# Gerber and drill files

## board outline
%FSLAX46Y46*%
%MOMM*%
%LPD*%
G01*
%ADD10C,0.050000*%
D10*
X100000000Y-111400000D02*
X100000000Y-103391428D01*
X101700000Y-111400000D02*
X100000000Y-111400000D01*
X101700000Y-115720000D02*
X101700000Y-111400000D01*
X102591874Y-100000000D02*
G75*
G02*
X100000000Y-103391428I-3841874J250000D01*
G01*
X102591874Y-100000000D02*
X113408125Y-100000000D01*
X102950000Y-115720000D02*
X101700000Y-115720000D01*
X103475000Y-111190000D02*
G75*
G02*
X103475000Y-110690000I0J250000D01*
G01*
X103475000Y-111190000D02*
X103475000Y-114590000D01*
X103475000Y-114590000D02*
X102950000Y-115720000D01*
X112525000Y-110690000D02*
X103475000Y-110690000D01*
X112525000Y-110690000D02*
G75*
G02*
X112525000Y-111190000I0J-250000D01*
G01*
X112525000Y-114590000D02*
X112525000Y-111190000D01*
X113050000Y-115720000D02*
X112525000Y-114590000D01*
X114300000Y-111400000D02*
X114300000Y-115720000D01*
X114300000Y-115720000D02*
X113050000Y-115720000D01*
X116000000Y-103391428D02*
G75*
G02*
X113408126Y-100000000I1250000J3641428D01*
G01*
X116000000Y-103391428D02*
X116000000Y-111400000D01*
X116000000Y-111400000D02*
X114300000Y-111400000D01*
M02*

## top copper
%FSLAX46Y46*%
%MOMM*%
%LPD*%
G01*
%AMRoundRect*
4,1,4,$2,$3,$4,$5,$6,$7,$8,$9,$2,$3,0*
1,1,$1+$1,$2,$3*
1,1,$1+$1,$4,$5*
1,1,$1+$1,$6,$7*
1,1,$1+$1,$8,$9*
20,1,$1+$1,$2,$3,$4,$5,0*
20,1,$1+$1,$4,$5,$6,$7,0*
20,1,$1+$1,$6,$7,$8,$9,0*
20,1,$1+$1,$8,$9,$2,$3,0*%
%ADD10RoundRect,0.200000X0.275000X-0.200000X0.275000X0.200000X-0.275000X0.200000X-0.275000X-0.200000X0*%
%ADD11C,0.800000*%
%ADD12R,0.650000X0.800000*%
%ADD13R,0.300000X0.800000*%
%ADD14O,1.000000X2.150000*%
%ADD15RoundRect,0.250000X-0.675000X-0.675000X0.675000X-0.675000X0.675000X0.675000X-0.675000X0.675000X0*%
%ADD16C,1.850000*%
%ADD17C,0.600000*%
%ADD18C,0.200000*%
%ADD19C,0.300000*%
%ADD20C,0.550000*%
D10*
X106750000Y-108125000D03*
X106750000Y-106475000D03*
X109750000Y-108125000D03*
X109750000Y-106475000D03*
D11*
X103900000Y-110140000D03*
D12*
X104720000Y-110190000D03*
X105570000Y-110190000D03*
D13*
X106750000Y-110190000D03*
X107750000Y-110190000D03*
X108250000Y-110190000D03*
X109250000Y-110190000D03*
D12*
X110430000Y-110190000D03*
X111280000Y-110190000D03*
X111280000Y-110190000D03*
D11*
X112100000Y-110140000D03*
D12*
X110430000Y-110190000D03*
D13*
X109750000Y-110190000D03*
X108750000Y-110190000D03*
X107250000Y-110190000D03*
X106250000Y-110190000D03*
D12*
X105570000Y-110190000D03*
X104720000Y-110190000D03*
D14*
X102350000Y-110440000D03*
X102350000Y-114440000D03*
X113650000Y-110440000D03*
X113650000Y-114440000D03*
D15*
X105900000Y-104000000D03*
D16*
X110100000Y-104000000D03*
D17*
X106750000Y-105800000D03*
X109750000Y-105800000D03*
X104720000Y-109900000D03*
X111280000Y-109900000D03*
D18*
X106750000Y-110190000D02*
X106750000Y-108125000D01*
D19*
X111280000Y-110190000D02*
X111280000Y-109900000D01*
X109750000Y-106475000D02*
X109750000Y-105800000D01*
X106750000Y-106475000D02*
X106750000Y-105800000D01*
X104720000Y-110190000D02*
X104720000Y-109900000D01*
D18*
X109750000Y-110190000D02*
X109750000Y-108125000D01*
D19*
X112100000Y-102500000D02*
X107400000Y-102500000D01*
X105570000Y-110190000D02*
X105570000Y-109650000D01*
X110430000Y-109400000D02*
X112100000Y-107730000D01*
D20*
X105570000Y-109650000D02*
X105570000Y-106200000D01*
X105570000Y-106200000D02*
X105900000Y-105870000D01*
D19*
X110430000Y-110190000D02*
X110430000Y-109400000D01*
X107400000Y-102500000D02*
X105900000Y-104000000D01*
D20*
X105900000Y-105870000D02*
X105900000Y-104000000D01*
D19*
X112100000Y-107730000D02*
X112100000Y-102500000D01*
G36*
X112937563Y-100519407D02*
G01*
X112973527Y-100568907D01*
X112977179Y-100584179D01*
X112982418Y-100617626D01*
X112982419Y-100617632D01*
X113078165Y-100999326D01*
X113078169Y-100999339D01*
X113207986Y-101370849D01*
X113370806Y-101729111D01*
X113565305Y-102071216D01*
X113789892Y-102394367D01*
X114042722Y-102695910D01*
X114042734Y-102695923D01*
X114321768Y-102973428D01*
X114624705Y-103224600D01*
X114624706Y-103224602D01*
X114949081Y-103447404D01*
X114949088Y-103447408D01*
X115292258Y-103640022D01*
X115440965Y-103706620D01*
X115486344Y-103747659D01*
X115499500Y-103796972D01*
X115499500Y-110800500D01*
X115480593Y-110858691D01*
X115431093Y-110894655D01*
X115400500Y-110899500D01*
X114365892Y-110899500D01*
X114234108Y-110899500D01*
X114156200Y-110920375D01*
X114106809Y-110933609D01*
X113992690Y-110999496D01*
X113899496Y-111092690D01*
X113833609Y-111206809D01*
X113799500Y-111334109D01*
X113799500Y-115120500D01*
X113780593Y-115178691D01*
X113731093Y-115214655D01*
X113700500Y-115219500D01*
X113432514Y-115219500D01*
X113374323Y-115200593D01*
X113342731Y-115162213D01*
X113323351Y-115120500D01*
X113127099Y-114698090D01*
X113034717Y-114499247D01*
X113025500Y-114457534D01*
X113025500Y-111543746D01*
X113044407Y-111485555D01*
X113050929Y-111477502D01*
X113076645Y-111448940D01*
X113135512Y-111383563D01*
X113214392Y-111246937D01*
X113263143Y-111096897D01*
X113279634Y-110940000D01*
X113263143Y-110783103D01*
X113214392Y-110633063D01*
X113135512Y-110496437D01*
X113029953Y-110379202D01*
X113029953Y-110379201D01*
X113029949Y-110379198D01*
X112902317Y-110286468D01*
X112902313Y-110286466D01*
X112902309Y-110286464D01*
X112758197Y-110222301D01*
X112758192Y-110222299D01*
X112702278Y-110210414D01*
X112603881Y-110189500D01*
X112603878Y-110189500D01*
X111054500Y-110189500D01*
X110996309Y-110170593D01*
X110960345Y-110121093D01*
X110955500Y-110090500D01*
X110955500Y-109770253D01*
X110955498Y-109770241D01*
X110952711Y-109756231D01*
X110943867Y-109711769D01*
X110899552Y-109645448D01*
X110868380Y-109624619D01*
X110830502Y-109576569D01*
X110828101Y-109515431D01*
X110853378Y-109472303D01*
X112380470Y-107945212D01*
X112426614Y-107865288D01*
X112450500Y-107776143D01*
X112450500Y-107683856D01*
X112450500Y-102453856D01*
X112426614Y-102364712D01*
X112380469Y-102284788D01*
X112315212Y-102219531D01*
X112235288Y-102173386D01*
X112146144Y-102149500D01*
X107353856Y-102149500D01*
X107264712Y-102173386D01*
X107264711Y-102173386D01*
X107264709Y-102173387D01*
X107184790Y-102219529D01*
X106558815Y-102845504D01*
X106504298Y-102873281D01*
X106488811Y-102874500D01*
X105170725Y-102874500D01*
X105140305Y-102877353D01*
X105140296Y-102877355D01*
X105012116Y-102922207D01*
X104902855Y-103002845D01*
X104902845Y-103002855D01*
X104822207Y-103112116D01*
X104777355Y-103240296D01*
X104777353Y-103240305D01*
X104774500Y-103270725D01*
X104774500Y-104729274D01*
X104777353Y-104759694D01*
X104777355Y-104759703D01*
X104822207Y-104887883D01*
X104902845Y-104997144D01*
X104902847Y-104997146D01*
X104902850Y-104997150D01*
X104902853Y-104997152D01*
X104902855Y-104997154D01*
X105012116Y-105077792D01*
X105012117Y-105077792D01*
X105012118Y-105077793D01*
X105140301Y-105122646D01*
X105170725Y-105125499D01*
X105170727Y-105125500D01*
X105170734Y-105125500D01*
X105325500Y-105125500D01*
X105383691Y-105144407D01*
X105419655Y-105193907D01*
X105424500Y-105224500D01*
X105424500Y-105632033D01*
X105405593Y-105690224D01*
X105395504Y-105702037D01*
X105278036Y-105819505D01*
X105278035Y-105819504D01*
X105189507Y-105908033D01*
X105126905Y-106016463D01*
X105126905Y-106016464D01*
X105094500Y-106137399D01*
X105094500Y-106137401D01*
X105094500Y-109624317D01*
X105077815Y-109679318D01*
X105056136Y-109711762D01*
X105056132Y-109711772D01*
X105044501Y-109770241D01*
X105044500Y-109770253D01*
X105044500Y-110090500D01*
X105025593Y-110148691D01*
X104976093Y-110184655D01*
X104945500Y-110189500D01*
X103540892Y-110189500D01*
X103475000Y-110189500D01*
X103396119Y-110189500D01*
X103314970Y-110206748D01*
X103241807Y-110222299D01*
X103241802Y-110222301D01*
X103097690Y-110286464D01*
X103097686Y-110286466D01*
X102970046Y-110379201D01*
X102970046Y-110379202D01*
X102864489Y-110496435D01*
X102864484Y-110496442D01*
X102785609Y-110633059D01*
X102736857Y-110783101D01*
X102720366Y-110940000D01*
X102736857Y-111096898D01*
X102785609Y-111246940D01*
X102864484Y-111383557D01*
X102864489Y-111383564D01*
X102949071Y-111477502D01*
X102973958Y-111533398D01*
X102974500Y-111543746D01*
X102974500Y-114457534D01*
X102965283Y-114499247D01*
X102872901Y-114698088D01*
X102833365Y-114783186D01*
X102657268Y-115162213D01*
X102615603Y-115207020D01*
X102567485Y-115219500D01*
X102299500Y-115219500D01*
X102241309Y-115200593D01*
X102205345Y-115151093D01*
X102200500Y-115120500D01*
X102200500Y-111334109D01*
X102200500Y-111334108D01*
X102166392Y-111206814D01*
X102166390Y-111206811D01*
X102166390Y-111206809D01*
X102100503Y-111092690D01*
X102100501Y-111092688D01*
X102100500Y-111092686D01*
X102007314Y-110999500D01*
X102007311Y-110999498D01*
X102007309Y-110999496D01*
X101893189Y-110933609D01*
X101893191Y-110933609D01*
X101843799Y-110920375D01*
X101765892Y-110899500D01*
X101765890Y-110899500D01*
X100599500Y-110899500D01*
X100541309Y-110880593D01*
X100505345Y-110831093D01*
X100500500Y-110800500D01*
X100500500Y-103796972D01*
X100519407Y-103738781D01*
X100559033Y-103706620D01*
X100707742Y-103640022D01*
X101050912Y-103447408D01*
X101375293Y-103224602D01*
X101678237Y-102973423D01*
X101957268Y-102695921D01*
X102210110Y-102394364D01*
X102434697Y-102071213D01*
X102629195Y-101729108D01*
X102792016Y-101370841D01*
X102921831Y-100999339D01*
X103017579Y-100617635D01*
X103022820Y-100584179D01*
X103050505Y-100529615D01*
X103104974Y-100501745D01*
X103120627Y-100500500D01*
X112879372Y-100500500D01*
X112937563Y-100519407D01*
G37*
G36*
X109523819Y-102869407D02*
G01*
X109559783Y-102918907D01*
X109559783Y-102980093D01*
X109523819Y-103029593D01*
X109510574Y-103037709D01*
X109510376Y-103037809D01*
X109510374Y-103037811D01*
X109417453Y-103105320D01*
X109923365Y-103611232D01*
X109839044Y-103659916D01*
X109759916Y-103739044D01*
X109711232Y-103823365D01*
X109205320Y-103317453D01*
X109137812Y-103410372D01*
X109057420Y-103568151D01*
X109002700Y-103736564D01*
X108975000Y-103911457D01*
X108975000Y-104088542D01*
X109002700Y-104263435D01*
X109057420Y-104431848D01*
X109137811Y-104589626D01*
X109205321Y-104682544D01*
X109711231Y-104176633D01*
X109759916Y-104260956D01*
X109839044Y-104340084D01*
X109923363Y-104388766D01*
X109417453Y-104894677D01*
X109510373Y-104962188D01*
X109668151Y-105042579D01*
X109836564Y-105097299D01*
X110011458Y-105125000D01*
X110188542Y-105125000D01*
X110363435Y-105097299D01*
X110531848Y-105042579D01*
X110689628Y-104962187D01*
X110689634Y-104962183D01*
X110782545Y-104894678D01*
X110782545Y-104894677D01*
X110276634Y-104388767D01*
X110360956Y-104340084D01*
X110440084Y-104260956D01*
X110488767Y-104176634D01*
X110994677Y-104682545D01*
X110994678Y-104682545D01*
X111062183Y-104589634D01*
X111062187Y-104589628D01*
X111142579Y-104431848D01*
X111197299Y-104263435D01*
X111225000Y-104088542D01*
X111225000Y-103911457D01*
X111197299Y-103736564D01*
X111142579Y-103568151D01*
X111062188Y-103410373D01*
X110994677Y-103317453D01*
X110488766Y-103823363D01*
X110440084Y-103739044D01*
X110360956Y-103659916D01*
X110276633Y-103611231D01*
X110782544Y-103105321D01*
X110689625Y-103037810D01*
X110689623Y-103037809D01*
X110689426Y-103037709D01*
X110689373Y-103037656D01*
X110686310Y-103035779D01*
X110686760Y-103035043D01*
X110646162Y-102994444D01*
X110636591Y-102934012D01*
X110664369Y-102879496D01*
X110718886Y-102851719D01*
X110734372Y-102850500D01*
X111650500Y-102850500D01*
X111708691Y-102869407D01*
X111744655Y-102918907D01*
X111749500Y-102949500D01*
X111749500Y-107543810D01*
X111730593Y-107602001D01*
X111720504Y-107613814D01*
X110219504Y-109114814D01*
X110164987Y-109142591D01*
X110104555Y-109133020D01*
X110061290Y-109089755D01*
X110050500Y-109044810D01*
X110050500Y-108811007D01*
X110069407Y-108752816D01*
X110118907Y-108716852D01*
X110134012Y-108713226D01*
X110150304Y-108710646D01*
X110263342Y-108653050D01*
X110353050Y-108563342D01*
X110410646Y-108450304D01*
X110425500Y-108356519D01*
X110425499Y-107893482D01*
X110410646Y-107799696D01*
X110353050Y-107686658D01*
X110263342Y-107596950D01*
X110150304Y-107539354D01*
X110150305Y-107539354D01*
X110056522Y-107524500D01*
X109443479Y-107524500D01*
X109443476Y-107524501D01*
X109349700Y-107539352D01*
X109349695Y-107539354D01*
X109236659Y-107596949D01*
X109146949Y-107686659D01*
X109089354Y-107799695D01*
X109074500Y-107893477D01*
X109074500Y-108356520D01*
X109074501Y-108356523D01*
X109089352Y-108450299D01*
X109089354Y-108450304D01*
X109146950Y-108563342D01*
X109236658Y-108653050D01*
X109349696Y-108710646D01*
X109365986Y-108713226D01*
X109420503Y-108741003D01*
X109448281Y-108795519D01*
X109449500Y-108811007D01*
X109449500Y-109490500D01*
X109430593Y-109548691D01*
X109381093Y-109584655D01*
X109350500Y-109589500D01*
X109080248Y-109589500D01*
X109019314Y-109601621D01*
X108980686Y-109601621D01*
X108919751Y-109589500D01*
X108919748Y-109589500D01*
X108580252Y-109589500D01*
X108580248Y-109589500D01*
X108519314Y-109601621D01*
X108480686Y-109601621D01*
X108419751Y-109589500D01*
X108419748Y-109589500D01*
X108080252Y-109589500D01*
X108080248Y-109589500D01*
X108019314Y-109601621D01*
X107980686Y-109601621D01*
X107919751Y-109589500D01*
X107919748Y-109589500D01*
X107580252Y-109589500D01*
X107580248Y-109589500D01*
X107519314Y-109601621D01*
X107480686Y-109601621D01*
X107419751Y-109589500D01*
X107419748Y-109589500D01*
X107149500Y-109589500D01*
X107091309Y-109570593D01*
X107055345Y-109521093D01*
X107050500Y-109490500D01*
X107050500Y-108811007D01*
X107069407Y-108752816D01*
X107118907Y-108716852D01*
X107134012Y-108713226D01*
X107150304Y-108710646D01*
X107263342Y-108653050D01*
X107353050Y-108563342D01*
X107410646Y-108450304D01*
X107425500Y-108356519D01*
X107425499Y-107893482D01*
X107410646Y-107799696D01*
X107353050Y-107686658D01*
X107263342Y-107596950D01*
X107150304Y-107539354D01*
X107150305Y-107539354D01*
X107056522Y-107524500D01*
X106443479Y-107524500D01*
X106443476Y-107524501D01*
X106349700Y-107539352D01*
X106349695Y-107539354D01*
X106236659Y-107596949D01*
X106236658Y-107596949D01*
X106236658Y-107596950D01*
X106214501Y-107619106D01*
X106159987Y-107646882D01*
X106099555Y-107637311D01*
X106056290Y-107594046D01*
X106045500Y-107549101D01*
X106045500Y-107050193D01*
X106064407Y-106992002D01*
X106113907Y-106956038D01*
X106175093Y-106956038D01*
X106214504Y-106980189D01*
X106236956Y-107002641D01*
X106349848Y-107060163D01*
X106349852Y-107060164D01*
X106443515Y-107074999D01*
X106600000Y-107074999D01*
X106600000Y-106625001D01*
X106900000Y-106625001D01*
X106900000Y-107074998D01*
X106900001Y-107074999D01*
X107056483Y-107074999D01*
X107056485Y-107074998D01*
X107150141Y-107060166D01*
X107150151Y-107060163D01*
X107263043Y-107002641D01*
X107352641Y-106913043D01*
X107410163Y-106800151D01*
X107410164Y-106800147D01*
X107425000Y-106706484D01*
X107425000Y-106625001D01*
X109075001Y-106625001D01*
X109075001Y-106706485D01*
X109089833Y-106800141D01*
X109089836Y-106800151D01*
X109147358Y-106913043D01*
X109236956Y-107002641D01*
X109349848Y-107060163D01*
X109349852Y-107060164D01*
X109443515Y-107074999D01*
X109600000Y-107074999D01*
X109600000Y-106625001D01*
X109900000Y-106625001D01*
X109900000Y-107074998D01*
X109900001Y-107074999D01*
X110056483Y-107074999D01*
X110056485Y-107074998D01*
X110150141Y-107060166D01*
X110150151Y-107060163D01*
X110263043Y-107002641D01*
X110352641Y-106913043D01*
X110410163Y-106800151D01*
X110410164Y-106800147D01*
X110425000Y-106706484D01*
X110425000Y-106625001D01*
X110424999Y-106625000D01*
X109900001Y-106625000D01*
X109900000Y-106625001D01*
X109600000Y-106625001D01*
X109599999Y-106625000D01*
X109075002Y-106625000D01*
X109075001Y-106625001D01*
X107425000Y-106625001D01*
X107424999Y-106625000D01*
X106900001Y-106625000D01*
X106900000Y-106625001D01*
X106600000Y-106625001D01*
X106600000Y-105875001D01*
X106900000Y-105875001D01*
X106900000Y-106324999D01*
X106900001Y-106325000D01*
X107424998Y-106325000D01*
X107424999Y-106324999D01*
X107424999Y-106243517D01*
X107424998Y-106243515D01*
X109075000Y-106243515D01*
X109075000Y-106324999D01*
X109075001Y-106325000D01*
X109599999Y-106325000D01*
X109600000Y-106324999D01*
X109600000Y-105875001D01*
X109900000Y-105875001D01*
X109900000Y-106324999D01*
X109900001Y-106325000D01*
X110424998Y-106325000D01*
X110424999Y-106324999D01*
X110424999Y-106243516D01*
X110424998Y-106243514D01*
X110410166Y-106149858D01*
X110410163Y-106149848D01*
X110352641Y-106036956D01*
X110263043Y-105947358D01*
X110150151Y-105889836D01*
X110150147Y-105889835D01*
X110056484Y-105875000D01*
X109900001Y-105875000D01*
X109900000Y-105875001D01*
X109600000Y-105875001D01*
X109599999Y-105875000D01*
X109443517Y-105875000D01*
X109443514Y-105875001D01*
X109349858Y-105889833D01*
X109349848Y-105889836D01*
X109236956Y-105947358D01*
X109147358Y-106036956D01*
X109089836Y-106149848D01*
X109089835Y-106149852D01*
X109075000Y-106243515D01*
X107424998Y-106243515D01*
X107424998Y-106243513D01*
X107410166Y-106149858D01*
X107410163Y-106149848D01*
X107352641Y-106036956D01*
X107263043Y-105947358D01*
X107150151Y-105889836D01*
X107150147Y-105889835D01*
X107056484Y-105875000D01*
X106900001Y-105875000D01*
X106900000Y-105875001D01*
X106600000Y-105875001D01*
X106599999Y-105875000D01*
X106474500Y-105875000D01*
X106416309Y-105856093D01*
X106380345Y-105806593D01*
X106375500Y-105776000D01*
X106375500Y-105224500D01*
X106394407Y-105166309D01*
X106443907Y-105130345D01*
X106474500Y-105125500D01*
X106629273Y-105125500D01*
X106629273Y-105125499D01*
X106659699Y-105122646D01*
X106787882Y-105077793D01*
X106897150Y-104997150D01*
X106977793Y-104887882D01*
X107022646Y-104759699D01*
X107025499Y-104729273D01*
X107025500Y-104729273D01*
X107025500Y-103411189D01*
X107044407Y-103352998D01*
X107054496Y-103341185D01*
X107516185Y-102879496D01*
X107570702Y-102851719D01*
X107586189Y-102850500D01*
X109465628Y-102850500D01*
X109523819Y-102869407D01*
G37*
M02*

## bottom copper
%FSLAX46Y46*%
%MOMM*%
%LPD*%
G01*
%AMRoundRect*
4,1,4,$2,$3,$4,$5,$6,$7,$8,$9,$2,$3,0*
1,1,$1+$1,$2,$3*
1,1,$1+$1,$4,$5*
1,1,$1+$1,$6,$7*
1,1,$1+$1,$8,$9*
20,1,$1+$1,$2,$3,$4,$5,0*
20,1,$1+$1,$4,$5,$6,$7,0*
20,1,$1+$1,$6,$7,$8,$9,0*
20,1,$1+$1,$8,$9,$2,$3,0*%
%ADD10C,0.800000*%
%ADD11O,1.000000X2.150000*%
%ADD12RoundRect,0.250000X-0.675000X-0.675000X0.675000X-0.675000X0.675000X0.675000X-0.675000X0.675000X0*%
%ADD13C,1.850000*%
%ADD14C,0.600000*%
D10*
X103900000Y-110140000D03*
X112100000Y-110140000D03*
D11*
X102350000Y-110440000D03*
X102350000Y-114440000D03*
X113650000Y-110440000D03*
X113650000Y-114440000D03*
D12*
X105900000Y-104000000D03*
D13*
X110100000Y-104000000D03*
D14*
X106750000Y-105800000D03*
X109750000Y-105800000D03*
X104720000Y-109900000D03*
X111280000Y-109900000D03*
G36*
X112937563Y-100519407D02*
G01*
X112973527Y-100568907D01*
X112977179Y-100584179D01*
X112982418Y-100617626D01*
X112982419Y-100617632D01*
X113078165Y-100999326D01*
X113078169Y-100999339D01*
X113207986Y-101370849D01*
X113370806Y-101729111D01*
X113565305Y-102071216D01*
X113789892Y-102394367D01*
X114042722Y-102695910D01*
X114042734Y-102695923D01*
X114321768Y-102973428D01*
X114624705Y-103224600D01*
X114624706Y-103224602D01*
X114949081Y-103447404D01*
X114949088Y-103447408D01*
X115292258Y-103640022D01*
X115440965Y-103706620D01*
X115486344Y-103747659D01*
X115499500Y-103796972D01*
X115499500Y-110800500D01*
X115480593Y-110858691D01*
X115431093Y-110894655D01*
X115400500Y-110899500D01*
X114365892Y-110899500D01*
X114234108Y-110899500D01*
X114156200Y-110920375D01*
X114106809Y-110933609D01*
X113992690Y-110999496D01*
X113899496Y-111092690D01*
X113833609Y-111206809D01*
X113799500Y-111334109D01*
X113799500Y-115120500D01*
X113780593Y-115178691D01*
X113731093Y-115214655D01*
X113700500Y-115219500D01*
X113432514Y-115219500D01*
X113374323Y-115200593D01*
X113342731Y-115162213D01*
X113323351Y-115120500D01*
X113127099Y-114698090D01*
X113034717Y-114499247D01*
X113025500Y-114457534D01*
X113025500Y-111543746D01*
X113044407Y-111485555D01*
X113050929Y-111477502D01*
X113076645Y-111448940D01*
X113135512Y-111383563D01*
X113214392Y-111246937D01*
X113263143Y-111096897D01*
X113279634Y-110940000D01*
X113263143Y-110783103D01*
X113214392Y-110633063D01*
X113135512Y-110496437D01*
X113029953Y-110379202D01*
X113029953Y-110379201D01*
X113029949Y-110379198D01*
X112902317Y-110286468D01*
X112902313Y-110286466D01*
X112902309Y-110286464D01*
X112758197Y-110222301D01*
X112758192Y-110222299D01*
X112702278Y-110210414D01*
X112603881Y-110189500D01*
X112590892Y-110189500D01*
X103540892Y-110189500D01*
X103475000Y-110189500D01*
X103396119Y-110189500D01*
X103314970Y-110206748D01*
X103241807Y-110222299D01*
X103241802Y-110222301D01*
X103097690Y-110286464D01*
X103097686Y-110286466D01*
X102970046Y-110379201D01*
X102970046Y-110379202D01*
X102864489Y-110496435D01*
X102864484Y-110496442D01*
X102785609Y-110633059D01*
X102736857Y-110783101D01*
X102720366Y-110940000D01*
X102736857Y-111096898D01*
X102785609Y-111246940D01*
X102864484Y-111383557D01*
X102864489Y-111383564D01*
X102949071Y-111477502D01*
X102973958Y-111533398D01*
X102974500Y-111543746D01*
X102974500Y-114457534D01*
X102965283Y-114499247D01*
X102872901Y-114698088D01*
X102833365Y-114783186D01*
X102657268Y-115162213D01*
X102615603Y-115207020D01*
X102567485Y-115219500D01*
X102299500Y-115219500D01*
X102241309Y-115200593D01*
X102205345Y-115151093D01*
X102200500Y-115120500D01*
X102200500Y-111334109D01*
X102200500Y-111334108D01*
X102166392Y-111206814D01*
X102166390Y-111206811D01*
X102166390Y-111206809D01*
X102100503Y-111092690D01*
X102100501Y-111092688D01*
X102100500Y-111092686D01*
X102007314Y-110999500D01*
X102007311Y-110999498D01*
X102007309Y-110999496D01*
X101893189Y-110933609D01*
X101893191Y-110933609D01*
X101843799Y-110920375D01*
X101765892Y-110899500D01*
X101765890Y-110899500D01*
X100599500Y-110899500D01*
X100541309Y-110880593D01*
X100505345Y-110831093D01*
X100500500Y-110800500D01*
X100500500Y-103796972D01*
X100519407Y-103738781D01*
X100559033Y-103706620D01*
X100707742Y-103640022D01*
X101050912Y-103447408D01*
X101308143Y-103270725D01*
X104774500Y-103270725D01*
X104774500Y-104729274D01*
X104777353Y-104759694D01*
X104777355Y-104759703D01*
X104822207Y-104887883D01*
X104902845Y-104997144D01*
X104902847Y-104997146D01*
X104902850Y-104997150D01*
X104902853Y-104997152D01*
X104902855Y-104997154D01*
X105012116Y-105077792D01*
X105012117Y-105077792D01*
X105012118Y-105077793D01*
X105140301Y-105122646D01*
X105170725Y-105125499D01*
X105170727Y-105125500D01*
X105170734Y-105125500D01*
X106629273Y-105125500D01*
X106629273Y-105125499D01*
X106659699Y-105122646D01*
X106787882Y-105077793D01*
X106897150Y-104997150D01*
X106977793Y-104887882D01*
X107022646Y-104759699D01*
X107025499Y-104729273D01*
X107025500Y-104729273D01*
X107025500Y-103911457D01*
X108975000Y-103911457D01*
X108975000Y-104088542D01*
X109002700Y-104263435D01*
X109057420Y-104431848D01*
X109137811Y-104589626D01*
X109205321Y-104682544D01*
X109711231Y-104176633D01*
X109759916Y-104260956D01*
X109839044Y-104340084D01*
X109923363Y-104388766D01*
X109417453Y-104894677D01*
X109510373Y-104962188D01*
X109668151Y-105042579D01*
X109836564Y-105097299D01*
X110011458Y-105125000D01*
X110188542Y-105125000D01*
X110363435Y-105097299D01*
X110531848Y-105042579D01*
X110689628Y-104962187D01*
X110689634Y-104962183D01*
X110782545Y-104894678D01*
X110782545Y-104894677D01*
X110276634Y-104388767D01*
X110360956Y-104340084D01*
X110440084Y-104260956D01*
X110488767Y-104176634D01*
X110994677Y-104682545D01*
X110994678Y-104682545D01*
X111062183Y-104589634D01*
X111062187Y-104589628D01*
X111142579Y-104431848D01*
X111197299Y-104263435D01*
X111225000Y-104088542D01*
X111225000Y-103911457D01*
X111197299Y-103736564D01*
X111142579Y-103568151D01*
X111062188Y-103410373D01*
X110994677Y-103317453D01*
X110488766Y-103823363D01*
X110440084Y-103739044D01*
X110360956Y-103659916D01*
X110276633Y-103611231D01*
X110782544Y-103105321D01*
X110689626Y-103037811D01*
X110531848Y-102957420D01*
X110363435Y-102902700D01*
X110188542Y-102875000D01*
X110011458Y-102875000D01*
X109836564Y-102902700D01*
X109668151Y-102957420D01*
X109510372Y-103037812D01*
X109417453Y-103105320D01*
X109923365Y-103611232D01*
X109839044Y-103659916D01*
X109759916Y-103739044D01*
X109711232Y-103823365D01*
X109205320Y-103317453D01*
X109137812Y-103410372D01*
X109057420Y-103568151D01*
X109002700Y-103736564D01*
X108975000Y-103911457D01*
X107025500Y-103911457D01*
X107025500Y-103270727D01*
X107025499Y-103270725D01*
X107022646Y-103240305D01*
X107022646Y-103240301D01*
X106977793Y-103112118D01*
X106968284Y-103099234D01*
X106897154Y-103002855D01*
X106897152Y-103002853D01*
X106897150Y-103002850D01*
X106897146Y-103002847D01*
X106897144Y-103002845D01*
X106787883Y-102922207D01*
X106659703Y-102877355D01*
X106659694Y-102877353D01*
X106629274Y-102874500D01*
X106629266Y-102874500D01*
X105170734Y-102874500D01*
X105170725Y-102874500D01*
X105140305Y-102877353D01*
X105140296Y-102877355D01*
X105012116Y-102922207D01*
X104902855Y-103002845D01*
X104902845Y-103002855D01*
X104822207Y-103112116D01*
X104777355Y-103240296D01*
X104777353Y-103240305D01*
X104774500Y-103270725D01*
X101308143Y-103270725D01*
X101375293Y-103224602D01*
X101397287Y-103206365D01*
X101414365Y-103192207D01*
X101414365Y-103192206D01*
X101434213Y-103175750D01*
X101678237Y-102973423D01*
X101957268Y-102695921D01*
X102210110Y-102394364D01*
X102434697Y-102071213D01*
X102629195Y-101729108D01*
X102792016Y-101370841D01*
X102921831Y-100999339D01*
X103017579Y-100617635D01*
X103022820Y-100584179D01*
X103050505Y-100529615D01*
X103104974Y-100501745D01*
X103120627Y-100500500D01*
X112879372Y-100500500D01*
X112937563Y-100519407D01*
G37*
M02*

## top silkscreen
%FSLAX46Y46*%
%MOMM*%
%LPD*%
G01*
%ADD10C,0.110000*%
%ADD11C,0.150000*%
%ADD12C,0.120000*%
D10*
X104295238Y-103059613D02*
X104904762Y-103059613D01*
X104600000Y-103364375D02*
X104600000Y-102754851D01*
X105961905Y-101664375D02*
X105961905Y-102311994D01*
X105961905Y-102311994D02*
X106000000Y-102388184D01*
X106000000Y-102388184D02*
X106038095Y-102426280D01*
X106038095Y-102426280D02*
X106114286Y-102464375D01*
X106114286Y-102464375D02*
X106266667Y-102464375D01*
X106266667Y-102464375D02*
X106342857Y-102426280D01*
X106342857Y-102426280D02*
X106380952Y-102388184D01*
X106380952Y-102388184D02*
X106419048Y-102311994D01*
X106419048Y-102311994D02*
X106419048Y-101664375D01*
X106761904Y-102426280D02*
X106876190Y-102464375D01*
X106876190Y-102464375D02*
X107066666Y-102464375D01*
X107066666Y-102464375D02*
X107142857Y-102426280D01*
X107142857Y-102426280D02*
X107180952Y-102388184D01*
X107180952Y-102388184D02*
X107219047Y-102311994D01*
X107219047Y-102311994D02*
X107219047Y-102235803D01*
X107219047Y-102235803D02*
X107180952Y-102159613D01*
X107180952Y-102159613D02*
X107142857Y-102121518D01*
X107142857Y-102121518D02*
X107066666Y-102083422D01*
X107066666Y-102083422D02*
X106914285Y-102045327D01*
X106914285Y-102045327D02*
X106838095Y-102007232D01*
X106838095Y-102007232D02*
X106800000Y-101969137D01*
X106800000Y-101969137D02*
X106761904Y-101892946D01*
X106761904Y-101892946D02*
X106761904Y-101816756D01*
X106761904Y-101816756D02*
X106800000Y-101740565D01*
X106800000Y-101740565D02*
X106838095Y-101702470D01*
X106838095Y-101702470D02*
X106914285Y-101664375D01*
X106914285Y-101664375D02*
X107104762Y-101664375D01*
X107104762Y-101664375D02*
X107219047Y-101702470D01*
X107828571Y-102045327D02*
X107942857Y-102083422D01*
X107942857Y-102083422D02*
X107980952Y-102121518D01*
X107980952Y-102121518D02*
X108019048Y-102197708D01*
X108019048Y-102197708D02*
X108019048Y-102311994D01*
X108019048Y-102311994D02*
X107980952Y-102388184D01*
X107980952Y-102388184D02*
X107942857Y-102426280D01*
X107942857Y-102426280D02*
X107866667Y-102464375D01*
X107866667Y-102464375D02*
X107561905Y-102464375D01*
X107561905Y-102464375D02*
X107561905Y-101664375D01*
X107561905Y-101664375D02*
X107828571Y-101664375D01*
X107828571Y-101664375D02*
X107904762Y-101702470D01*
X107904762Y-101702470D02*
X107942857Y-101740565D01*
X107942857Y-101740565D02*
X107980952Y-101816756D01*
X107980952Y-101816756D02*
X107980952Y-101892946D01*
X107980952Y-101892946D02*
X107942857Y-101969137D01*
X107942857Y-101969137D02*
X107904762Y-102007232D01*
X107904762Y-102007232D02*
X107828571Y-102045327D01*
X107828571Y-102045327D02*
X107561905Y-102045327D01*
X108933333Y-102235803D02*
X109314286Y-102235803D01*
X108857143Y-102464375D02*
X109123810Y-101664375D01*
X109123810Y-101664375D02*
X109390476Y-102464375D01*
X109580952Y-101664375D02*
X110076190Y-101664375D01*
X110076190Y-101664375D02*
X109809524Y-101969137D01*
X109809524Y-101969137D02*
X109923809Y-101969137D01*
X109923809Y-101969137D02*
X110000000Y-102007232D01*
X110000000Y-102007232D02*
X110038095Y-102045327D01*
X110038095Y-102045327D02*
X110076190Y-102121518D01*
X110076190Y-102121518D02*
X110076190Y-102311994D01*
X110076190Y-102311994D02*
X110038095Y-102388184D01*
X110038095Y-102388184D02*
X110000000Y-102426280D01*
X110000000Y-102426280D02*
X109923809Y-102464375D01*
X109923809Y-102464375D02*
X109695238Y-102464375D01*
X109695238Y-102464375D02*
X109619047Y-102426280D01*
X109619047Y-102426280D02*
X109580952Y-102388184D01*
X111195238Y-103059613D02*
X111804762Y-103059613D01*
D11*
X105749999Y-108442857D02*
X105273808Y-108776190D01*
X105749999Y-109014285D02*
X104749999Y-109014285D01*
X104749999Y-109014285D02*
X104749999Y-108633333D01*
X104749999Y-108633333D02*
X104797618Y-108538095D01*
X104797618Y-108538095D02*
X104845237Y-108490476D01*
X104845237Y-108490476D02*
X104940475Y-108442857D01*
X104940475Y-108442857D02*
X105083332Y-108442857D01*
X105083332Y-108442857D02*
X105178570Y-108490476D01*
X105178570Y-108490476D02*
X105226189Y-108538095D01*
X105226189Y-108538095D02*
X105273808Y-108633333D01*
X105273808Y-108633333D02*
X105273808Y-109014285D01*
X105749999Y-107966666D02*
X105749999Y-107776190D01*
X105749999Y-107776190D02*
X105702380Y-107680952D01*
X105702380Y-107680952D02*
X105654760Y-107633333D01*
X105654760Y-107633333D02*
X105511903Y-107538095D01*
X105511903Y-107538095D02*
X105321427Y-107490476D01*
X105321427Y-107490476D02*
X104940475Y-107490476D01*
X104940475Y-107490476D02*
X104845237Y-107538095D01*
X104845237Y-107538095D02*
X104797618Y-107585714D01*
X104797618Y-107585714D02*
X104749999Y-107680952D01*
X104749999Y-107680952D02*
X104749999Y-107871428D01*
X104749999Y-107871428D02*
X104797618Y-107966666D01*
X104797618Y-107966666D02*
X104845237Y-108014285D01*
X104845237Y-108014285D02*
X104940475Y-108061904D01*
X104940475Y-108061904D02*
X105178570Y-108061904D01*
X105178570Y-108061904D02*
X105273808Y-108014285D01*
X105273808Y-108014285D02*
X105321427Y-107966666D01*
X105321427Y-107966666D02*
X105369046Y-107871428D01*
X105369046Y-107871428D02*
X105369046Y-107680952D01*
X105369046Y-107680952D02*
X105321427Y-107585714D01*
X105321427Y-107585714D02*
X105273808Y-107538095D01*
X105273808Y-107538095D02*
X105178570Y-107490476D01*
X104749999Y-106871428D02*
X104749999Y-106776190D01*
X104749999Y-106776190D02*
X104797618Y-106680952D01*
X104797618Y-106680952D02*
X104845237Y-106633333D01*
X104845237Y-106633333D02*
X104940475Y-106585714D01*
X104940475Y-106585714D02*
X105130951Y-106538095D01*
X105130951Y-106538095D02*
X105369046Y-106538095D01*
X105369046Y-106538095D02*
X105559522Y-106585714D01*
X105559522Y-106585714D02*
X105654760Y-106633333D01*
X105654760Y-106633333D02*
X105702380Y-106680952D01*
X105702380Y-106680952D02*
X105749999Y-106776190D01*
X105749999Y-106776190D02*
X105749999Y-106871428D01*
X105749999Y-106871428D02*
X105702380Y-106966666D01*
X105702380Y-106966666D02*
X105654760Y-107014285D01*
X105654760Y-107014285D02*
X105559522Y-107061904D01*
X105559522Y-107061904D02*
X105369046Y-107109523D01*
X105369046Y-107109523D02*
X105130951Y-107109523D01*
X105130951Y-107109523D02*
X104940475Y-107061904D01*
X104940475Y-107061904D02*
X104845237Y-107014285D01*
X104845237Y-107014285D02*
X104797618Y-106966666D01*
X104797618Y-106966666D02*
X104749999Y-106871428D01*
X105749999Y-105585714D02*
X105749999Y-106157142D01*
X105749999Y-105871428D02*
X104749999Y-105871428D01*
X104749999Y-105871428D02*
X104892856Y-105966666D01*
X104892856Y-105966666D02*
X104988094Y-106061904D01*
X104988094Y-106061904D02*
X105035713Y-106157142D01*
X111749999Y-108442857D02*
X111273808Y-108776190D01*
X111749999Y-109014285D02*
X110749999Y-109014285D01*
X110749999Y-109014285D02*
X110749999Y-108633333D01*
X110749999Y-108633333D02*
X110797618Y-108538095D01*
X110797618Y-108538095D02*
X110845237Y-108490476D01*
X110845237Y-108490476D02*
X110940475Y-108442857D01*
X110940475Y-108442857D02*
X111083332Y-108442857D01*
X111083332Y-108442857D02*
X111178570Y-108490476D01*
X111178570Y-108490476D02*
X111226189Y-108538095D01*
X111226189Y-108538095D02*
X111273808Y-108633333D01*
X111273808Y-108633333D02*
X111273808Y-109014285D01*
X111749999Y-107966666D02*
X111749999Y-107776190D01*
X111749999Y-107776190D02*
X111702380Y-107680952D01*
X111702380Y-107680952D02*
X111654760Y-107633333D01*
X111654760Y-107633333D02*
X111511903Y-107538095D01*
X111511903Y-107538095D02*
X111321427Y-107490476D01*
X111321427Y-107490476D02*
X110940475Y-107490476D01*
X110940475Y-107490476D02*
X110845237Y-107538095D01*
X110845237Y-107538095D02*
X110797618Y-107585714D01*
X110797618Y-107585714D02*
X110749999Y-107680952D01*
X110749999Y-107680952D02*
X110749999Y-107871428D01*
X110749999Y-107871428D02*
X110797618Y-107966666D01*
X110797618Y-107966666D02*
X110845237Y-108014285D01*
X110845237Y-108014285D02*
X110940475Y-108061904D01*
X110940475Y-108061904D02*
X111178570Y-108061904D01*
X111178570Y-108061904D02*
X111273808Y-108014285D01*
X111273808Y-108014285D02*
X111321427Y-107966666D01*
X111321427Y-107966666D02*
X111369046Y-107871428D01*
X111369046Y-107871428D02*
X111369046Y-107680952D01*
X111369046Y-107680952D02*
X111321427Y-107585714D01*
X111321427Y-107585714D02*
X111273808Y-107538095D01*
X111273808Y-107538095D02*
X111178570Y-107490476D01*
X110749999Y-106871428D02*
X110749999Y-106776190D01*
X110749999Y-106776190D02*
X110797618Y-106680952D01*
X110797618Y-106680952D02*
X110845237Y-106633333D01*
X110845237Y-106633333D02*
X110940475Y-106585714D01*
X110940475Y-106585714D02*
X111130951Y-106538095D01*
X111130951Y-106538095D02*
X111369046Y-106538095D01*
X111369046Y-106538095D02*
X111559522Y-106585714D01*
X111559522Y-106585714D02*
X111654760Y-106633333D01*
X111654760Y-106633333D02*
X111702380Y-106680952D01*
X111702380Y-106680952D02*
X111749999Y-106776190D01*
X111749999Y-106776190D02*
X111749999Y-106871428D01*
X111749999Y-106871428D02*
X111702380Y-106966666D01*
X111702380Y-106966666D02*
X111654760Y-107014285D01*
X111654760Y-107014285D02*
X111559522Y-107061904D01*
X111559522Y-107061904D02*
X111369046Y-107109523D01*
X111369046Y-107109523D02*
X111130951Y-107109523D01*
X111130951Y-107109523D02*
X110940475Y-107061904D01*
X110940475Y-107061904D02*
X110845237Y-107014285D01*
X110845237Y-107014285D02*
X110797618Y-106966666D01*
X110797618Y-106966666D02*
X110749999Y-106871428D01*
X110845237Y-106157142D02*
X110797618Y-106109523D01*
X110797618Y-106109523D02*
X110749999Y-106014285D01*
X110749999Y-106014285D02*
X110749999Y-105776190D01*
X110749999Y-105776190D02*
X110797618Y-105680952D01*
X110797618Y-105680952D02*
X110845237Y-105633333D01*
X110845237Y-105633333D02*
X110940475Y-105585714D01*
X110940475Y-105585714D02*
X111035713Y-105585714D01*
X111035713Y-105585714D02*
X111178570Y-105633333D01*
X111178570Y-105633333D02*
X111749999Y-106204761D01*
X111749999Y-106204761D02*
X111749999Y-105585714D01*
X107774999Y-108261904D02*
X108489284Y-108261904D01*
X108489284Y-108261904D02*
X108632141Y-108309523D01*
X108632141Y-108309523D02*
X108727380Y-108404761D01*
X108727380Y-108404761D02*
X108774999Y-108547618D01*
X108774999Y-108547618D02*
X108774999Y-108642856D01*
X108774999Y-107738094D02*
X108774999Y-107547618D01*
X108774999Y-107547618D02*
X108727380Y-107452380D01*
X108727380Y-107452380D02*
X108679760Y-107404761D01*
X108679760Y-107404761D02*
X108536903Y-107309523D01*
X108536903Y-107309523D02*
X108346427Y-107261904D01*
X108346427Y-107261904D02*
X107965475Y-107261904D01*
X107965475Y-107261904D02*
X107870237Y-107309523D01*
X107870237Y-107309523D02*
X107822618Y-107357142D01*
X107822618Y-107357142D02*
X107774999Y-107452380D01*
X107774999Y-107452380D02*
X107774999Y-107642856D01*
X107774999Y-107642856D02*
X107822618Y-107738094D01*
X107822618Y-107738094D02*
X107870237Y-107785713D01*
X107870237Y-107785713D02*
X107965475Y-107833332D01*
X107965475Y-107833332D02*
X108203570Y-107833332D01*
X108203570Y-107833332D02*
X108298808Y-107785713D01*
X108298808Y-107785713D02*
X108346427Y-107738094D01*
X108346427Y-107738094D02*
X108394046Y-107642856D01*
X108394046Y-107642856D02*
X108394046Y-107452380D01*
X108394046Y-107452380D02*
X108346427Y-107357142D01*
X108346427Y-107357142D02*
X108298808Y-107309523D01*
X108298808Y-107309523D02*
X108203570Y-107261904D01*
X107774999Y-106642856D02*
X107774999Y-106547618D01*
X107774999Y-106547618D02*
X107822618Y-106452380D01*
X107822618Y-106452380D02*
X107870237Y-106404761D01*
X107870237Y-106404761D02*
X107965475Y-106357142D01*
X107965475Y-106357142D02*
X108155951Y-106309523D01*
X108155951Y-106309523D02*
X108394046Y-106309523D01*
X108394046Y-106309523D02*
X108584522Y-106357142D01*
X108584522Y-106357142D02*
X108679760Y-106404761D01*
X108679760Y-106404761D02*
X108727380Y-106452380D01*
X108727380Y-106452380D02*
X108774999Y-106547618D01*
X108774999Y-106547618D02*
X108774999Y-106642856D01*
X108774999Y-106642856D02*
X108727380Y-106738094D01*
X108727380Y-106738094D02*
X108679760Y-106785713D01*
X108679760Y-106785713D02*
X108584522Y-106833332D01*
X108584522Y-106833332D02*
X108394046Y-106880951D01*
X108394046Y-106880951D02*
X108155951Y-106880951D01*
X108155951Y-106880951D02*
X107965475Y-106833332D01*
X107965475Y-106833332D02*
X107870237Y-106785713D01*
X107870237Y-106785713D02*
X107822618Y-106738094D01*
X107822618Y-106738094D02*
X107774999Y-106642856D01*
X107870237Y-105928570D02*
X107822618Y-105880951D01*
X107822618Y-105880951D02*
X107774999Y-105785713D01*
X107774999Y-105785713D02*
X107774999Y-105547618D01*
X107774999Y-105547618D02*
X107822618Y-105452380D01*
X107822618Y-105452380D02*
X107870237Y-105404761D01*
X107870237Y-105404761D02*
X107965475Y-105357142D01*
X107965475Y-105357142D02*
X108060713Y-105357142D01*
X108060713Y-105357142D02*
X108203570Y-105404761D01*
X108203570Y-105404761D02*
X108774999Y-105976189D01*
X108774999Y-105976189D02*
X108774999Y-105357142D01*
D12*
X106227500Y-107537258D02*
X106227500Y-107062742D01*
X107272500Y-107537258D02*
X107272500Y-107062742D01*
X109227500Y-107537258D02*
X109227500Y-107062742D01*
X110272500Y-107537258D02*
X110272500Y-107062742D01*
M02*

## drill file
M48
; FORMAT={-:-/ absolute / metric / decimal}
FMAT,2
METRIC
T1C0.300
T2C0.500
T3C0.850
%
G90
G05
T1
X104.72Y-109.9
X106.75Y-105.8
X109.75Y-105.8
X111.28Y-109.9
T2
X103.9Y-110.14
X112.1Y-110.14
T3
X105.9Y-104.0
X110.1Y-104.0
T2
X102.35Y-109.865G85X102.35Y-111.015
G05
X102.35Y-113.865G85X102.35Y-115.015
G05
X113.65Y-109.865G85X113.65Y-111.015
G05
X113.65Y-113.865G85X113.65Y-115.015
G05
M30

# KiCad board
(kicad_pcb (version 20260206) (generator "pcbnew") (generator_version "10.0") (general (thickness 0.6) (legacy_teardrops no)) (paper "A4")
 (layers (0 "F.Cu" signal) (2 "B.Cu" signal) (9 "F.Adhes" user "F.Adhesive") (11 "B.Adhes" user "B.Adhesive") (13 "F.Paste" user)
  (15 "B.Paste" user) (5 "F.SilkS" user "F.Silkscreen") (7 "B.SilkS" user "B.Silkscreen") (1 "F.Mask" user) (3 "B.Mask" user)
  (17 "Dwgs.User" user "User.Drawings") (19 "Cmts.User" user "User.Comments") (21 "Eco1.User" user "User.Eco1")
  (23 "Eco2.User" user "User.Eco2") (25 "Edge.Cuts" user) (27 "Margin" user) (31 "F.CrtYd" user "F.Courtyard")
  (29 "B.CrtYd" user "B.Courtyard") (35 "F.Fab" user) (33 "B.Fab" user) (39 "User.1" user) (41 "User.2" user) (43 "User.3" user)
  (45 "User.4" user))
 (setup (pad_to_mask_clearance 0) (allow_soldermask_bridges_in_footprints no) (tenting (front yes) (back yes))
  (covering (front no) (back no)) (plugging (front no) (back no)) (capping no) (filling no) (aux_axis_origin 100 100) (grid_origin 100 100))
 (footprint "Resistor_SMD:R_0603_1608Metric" (layer "F.Cu") (at 106.75 107.3 90)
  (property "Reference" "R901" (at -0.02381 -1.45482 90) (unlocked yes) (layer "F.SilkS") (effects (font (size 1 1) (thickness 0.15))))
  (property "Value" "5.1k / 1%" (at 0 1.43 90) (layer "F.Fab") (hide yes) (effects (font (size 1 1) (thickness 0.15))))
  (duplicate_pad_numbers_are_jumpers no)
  (fp_line (start -0.237258 -0.5225) (end 0.237258 -0.5225) (stroke (width 0.12) (type solid)) (layer "F.SilkS"))
  (fp_line (start -0.237258 0.5225) (end 0.237258 0.5225) (stroke (width 0.12) (type solid)) (layer "F.SilkS"))
  (pad "1" smd roundrect (at -0.825 0 90) (size 0.8 0.95) (layers "F.Cu" "F.Mask" "F.Paste") (roundrect_rratio 0.25) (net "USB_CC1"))
  (pad "2" smd roundrect (at 0.825 0 90) (size 0.8 0.95) (layers "F.Cu" "F.Mask" "F.Paste") (roundrect_rratio 0.25) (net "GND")))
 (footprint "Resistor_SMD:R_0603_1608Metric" (layer "F.Cu") (at 109.75 107.3 90)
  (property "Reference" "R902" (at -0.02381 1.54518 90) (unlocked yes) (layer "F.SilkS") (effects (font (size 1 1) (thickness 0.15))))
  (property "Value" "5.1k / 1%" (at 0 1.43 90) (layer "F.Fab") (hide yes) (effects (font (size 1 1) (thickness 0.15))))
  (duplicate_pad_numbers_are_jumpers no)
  (fp_line (start -0.237258 -0.5225) (end 0.237258 -0.5225) (stroke (width 0.12) (type solid)) (layer "F.SilkS"))
  (fp_line (start -0.237258 0.5225) (end 0.237258 0.5225) (stroke (width 0.12) (type solid)) (layer "F.SilkS"))
  (pad "1" smd roundrect (at -0.825 0 90) (size 0.8 0.95) (layers "F.Cu" "F.Mask" "F.Paste") (roundrect_rratio 0.25) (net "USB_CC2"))
  (pad "2" smd roundrect (at 0.825 0 90) (size 0.8 0.95) (layers "F.Cu" "F.Mask" "F.Paste") (roundrect_rratio 0.25) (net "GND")))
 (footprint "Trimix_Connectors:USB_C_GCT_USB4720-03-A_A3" (layer "F.Cu") (at 108 110.14)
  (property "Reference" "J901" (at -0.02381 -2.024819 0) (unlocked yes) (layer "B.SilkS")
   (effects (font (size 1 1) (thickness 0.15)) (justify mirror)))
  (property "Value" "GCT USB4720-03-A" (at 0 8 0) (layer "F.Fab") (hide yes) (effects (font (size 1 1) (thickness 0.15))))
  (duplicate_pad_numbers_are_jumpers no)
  (pad "A1" thru_hole circle (at -4.1 0) (size 0.8 0.8) (drill 0.5) (layers "*.Cu" "*.Mask") (remove_unused_layers no) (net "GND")
   (zone_connect 2))
  (pad "A1" smd rect (at -3.28 0.05) (size 0.65 0.8) (layers "F.Cu" "F.Mask" "F.Paste") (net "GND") (zone_connect 2))
  (pad "A4" smd rect (at -2.43 0.05) (size 0.65 0.8) (layers "F.Cu" "F.Mask" "F.Paste") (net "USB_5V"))
  (pad "A5" smd rect (at -1.25 0.05) (size 0.3 0.8) (layers "F.Cu" "F.Mask" "F.Paste") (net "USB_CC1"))
  (pad "A6" smd rect (at -0.25 0.05) (size 0.3 0.8) (layers "F.Cu" "F.Mask" "F.Paste") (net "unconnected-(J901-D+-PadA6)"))
  (pad "A7" smd rect (at 0.25 0.05) (size 0.3 0.8) (layers "F.Cu" "F.Mask" "F.Paste") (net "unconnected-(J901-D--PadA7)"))
  (pad "A8" smd rect (at 1.25 0.05) (size 0.3 0.8) (layers "F.Cu" "F.Mask" "F.Paste") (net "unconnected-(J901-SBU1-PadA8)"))
  (pad "A9" smd rect (at 2.43 0.05) (size 0.65 0.8) (layers "F.Cu" "F.Mask" "F.Paste") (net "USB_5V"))
  (pad "A12" smd rect (at 3.28 0.05) (size 0.65 0.8) (layers "F.Cu" "F.Mask" "F.Paste") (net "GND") (zone_connect 2))
  (pad "B1" smd rect (at 3.28 0.05) (size 0.65 0.8) (layers "F.Cu" "F.Mask" "F.Paste") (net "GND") (zone_connect 2))
  (pad "B1" thru_hole circle (at 4.1 0) (size 0.8 0.8) (drill 0.5) (layers "*.Cu" "*.Mask") (remove_unused_layers no) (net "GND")
   (zone_connect 2))
  (pad "B4" smd rect (at 2.43 0.05) (size 0.65 0.8) (layers "F.Cu" "F.Mask" "F.Paste") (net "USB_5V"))
  (pad "B5" smd rect (at 1.75 0.05) (size 0.3 0.8) (layers "F.Cu" "F.Mask" "F.Paste") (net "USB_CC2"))
  (pad "B6" smd rect (at 0.75 0.05) (size 0.3 0.8) (layers "F.Cu" "F.Mask" "F.Paste") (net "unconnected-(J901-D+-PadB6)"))
  (pad "B7" smd rect (at -0.75 0.05) (size 0.3 0.8) (layers "F.Cu" "F.Mask" "F.Paste") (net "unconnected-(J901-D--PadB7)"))
  (pad "B8" smd rect (at -1.75 0.05) (size 0.3 0.8) (layers "F.Cu" "F.Mask" "F.Paste") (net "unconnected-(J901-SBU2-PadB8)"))
  (pad "B9" smd rect (at -2.43 0.05) (size 0.65 0.8) (layers "F.Cu" "F.Mask" "F.Paste") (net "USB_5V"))
  (pad "B12" smd rect (at -3.28 0.05) (size 0.65 0.8) (layers "F.Cu" "F.Mask" "F.Paste") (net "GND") (zone_connect 2))
  (pad "SH" thru_hole oval (at -5.65 0.3) (size 1 2.15) (drill oval 0.5 1.65) (layers "*.Cu" "*.Mask") (remove_unused_layers no) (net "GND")
   (zone_connect 2))
  (pad "SH" thru_hole oval (at -5.65 4.3) (size 1 2.15) (drill oval 0.5 1.65) (layers "*.Cu" "*.Mask") (remove_unused_layers no) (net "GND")
   (zone_connect 2))
  (pad "SH" thru_hole oval (at 5.65 0.3) (size 1 2.15) (drill oval 0.5 1.65) (layers "*.Cu" "*.Mask") (remove_unused_layers no) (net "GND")
   (zone_connect 2))
  (pad "SH" thru_hole oval (at 5.65 4.3) (size 1 2.15) (drill oval 0.5 1.65) (layers "*.Cu" "*.Mask") (remove_unused_layers no) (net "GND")
   (zone_connect 2)))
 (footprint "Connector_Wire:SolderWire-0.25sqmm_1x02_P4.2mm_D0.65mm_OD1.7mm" (layer "F.Cu") (at 105.9 104)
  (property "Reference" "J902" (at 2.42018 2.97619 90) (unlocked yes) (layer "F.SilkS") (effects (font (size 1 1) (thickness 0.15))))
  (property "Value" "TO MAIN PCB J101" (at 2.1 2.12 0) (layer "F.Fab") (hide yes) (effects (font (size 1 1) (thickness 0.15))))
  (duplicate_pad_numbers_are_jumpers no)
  (pad "1" thru_hole roundrect (at 0 0) (size 1.85 1.85) (drill 0.85) (layers "*.Cu" "*.Mask") (remove_unused_layers no)
   (roundrect_rratio 0.135135) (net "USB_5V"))
  (pad "2" thru_hole circle (at 4.2 0) (size 1.85 1.85) (drill 0.85) (layers "*.Cu" "*.Mask") (remove_unused_layers no) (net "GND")))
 (gr_line (start 100 111.4) (end 100 103.391428) (stroke (width 0.05) (type default)) (layer "Edge.Cuts"))
 (gr_line (start 101.7 111.4) (end 100 111.4) (stroke (width 0.05) (type default)) (layer "Edge.Cuts"))
 (gr_line (start 101.7 115.72) (end 101.7 111.4) (stroke (width 0.05) (type default)) (layer "Edge.Cuts"))
 (gr_arc (start 102.591874 100) (mid 101.808961 102.087789) (end 100 103.391428) (stroke (width 0.05) (type default)) (layer "Edge.Cuts"))
 (gr_line (start 102.591874 100) (end 113.408125 100) (stroke (width 0.05) (type default)) (layer "Edge.Cuts"))
 (gr_line (start 102.95 115.72) (end 101.7 115.72) (stroke (width 0.05) (type default)) (layer "Edge.Cuts"))
 (gr_arc (start 103.475 111.19) (mid 103.225 110.94) (end 103.475 110.69) (stroke (width 0.05) (type default)) (layer "Edge.Cuts"))
 (gr_line (start 103.475 111.19) (end 103.475 114.59) (stroke (width 0.05) (type default)) (layer "Edge.Cuts"))
 (gr_line (start 103.475 114.59) (end 102.95 115.72) (stroke (width 0.05) (type default)) (layer "Edge.Cuts"))
 (gr_line (start 112.525 110.69) (end 103.475 110.69) (stroke (width 0.05) (type default)) (layer "Edge.Cuts"))
 (gr_arc (start 112.525 110.69) (mid 112.775 110.94) (end 112.525 111.19) (stroke (width 0.05) (type default)) (layer "Edge.Cuts"))
 (gr_line (start 112.525 114.59) (end 112.525 111.19) (stroke (width 0.05) (type default)) (layer "Edge.Cuts"))
 (gr_line (start 113.05 115.72) (end 112.525 114.59) (stroke (width 0.05) (type default)) (layer "Edge.Cuts"))
 (gr_line (start 114.3 111.4) (end 114.3 115.72) (stroke (width 0.05) (type default)) (layer "Edge.Cuts"))
 (gr_line (start 114.3 115.72) (end 113.05 115.72) (stroke (width 0.05) (type default)) (layer "Edge.Cuts"))
 (gr_arc (start 116 103.391428) (mid 114.191039 102.087789) (end 113.408125 100) (stroke (width 0.05) (type default)) (layer "Edge.Cuts"))
 (gr_line (start 116 103.391428) (end 116 111.4) (stroke (width 0.05) (type default)) (layer "Edge.Cuts"))
 (gr_line (start 116 111.4) (end 114.3 111.4) (stroke (width 0.05) (type default)) (layer "Edge.Cuts"))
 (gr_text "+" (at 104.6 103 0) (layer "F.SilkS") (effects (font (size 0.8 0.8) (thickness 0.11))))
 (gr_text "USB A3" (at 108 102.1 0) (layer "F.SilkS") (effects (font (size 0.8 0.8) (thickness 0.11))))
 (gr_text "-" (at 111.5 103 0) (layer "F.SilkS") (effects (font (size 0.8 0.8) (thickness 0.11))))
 (segment (start 106.75 110.19) (end 106.75 108.125) (width 0.2) (layer "F.Cu") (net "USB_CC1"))
 (segment (start 111.28 110.19) (end 111.28 109.9) (width 0.3) (layer "F.Cu") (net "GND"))
 (segment (start 109.75 106.475) (end 109.75 105.8) (width 0.3) (layer "F.Cu") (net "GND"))
 (segment (start 106.75 106.475) (end 106.75 105.8) (width 0.3) (layer "F.Cu") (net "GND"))
 (segment (start 104.72 110.19) (end 104.72 109.9) (width 0.3) (layer "F.Cu") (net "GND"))
 (via (at 106.75 105.8) (size 0.6) (drill 0.3) (layers "F.Cu" "B.Cu") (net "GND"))
 (via (at 109.75 105.8) (size 0.6) (drill 0.3) (layers "F.Cu" "B.Cu") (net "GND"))
 (via (at 104.72 109.9) (size 0.6) (drill 0.3) (layers "F.Cu" "B.Cu") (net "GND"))
 (via (at 111.28 109.9) (size 0.6) (drill 0.3) (layers "F.Cu" "B.Cu") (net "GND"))
 (segment (start 109.75 110.19) (end 109.75 108.125) (width 0.2) (layer "F.Cu") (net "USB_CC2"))
 (segment (start 112.1 102.5) (end 107.4 102.5) (width 0.3) (layer "F.Cu") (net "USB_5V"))
 (segment (start 105.57 110.19) (end 105.57 109.65) (width 0.3) (layer "F.Cu") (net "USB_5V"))
 (segment (start 110.43 109.4) (end 112.1 107.73) (width 0.3) (layer "F.Cu") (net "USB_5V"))
 (segment (start 105.57 109.65) (end 105.57 106.2) (width 0.55) (layer "F.Cu") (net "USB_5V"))
 (segment (start 105.57 106.2) (end 105.9 105.87) (width 0.55) (layer "F.Cu") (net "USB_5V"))
 (segment (start 110.43 110.19) (end 110.43 109.4) (width 0.3) (layer "F.Cu") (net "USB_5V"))
 (segment (start 107.4 102.5) (end 105.9 104) (width 0.3) (layer "F.Cu") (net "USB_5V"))
 (segment (start 105.9 105.87) (end 105.9 104) (width 0.55) (layer "F.Cu") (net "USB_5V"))
 (segment (start 112.1 107.73) (end 112.1 102.5) (width 0.3) (layer "F.Cu") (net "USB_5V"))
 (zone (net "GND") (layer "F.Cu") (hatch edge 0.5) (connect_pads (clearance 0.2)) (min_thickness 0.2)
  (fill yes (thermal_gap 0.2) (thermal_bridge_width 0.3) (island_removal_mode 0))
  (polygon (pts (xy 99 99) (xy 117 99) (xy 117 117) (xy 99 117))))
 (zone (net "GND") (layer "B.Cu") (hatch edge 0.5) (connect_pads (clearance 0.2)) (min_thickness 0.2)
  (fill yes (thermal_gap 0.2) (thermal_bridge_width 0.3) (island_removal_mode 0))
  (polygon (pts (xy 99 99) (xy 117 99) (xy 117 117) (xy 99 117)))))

